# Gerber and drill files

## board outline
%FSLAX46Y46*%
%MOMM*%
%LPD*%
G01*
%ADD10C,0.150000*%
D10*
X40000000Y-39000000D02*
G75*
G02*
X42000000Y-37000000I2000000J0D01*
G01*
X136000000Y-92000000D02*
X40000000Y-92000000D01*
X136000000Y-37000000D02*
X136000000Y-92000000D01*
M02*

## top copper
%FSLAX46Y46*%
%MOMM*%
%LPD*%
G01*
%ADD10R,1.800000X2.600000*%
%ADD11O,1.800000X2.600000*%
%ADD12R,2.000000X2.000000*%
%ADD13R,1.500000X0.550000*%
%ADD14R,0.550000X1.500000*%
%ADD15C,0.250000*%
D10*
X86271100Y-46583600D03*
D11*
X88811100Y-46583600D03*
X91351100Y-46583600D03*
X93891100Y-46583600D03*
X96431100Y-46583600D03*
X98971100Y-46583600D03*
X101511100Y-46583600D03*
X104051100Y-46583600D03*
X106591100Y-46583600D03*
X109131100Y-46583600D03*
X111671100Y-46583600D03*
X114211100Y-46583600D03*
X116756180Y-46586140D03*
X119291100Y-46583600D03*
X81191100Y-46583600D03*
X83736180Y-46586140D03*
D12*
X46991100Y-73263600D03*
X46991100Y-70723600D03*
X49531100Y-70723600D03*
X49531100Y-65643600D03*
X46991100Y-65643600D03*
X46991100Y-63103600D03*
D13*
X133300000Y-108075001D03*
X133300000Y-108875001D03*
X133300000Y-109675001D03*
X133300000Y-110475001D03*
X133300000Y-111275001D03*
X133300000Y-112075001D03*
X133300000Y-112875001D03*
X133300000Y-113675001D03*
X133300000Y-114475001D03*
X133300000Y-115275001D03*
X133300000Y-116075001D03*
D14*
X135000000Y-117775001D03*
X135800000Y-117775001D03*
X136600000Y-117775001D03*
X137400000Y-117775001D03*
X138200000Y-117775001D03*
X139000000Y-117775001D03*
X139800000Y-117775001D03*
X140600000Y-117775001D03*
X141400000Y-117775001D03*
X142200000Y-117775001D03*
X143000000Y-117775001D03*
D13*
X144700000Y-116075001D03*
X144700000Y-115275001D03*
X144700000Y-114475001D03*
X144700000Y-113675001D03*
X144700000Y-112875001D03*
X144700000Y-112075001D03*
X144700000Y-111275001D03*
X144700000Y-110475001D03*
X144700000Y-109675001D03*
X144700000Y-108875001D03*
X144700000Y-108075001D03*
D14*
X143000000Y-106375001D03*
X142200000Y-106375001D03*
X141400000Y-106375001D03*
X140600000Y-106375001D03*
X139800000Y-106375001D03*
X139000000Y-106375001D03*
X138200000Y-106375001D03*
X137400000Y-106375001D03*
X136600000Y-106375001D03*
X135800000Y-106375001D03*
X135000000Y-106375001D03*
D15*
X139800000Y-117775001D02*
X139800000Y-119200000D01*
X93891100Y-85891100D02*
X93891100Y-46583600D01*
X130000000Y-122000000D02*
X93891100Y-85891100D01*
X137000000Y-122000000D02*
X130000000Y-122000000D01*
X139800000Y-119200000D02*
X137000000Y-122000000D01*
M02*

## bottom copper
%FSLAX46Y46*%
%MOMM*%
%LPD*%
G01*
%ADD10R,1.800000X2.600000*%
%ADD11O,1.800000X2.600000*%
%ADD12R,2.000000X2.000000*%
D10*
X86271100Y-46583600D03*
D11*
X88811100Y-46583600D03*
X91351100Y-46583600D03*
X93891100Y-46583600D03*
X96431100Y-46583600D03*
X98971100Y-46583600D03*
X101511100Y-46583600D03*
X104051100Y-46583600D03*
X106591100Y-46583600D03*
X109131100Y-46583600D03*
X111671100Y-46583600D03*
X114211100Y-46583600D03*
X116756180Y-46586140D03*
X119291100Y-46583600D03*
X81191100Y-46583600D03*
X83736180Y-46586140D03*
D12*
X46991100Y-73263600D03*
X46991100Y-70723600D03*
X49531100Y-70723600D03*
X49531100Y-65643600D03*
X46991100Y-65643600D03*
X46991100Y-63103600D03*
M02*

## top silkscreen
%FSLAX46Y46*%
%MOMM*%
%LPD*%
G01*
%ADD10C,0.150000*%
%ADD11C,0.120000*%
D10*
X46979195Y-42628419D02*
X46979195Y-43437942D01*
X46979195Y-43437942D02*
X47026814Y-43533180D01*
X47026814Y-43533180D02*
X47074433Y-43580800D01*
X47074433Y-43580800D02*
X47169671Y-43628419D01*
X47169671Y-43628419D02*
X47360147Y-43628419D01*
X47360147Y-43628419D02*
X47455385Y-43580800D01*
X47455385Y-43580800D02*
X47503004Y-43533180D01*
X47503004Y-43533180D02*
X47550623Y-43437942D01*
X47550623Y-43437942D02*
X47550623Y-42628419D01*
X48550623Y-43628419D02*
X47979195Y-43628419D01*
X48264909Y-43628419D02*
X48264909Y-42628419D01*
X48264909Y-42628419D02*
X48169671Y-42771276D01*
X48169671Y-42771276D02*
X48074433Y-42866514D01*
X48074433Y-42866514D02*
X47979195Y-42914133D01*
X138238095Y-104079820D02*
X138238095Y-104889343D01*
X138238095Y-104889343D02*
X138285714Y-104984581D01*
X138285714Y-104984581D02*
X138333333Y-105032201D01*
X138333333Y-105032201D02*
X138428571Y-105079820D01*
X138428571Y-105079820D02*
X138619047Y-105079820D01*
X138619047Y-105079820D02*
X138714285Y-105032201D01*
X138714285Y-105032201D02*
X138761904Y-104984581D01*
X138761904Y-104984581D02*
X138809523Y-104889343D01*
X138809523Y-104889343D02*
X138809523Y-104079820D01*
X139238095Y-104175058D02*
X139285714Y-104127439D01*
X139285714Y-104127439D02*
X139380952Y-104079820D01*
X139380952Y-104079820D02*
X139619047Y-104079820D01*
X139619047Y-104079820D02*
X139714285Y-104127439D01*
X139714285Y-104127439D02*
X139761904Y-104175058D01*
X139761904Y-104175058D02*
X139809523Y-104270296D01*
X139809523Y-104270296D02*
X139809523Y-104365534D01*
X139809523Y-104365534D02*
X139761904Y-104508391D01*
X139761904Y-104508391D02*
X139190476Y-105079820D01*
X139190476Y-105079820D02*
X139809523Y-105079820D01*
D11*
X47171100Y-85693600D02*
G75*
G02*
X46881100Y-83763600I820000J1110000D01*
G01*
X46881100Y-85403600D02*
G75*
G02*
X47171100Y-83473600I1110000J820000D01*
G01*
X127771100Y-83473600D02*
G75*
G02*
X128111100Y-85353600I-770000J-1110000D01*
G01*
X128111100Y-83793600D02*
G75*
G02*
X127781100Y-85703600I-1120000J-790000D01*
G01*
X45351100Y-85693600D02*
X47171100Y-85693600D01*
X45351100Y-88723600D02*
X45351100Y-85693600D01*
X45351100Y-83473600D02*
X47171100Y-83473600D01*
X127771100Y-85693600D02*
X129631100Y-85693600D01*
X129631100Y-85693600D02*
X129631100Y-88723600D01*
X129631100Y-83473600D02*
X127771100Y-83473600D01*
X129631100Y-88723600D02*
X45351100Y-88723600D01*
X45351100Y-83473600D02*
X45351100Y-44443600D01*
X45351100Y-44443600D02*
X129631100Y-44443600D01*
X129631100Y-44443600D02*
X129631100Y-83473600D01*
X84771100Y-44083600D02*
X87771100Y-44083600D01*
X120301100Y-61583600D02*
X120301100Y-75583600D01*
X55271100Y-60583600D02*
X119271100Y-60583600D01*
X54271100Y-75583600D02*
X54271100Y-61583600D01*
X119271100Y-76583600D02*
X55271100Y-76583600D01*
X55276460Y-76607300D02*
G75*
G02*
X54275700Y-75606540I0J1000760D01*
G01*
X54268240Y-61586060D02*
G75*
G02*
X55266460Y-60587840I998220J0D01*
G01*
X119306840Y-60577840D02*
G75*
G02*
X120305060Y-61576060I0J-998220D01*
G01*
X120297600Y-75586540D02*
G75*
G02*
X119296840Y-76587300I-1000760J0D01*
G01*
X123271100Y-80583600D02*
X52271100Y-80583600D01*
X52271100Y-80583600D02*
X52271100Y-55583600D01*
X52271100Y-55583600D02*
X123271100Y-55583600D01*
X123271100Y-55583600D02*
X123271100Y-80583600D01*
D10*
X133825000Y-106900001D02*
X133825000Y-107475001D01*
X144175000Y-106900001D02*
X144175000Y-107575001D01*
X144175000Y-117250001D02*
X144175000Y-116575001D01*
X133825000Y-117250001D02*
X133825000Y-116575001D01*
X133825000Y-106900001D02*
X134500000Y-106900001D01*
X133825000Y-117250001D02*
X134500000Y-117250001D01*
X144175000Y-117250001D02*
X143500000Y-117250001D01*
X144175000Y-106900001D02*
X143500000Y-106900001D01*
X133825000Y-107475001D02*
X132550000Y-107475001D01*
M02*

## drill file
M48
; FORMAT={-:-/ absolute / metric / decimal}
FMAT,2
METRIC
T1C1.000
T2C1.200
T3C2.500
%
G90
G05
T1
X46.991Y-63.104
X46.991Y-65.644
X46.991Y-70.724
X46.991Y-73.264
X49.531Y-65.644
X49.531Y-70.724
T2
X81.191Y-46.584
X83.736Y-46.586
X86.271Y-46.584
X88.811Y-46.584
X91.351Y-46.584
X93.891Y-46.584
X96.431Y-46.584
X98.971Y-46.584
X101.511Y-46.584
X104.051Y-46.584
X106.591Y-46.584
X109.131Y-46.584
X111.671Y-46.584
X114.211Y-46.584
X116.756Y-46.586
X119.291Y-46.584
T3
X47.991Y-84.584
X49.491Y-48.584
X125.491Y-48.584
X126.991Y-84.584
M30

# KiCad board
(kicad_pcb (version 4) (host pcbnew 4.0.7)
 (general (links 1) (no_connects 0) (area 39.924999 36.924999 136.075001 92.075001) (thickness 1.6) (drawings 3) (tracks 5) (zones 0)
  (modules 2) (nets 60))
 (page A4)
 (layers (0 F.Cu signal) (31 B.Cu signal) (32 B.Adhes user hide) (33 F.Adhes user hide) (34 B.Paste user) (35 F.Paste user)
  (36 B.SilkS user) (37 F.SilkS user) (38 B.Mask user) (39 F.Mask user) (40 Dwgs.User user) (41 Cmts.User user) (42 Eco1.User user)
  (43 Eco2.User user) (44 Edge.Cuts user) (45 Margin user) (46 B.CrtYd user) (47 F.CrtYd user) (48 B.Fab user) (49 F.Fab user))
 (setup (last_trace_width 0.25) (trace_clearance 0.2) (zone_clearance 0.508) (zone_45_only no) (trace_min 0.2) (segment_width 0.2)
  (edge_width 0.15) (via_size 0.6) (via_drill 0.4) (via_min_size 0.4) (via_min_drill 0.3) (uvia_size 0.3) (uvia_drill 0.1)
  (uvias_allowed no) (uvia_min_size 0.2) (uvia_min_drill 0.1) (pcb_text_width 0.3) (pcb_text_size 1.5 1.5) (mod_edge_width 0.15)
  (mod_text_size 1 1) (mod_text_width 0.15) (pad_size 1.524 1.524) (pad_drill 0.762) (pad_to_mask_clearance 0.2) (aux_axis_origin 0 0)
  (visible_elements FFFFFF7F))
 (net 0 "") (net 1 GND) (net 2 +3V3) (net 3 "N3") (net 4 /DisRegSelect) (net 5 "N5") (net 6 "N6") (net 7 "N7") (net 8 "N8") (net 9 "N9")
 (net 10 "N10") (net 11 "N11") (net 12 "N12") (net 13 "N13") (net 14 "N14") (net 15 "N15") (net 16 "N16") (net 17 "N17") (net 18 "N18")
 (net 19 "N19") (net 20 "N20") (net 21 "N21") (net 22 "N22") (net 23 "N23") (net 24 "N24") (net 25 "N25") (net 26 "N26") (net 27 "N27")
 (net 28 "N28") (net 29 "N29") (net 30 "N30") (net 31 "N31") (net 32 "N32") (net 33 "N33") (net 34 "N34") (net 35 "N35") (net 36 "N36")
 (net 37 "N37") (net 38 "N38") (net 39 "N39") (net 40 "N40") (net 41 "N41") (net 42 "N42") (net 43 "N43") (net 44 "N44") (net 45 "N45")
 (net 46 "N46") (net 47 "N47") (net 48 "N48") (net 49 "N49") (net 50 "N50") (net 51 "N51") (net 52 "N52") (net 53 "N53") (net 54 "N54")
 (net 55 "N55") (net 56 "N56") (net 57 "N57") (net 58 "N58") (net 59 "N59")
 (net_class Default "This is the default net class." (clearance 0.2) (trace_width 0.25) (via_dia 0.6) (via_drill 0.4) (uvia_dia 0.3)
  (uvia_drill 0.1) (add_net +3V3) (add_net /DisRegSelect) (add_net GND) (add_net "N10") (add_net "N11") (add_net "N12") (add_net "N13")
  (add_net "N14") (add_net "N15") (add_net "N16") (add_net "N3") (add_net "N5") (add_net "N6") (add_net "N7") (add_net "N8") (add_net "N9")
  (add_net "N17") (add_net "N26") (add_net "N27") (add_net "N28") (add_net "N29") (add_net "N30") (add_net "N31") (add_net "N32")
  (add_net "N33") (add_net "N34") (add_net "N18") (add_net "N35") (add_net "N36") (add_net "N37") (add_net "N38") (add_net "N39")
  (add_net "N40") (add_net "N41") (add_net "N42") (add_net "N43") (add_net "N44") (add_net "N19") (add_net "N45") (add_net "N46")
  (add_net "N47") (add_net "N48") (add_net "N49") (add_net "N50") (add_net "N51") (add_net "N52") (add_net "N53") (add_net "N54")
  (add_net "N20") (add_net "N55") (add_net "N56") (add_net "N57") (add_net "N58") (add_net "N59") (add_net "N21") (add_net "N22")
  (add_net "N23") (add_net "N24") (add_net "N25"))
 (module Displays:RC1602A (layer F.Cu) (at 86.2711 46.5836)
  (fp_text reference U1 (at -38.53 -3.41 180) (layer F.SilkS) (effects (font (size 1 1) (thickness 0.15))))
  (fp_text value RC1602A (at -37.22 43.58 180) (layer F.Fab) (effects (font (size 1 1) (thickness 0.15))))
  (fp_arc (start -38.28 38) (end -39.1 39.11) (angle 90) (layer F.SilkS) (width 0.12))
  (fp_arc (start -38.28 38) (end -39.39 38.82) (angle 90) (layer F.SilkS) (width 0.12))
  (fp_arc (start 40.73 38) (end 41.5 36.89) (angle 90) (layer F.SilkS) (width 0.12))
  (fp_arc (start 40.72 38) (end 41.84 37.21) (angle 90) (layer F.SilkS) (width 0.12))
  (fp_line (start -40.92 39.11) (end -39.1 39.11) (layer F.SilkS) (width 0.12))
  (fp_line (start -40.92 42.14) (end -40.92 39.11) (layer F.SilkS) (width 0.12))
  (fp_line (start -40.92 36.89) (end -39.1 36.89) (layer F.SilkS) (width 0.12))
  (fp_line (start 41.5 39.11) (end 43.36 39.11) (layer F.SilkS) (width 0.12))
  (fp_line (start 43.36 39.11) (end 43.36 42.14) (layer F.SilkS) (width 0.12))
  (fp_line (start 43.36 36.89) (end 41.5 36.89) (layer F.SilkS) (width 0.12))
  (fp_line (start 43.36 42.14) (end -40.92 42.14) (layer F.SilkS) (width 0.12))
  (fp_line (start -40.92 36.89) (end -40.92 -2.14) (layer F.SilkS) (width 0.12))
  (fp_line (start -40.92 -2.14) (end 43.36 -2.14) (layer F.SilkS) (width 0.12))
  (fp_line (start 43.36 -2.14) (end 43.36 36.89) (layer F.SilkS) (width 0.12))
  (fp_line (start -1.5 -2.5) (end 1.5 -2.5) (layer F.SilkS) (width 0.12))
  (fp_line (start 34.03 15) (end 34.03 29) (layer F.SilkS) (width 0.12))
  (fp_line (start -31 14) (end 33 14) (layer F.SilkS) (width 0.12))
  (fp_line (start -32 29) (end -32 15) (layer F.SilkS) (width 0.12))
  (fp_line (start 33 30) (end -31 30) (layer F.SilkS) (width 0.12))
  (fp_arc (start -30.99464 29.02294) (end -30.99464 30.0237) (angle 90) (layer F.SilkS) (width 0.12))
  (fp_arc (start -31.00464 15.00246) (end -32.00286 15.00246) (angle 90) (layer F.SilkS) (width 0.12))
  (fp_arc (start 33.03574 14.99246) (end 33.03574 13.99424) (angle 90) (layer F.SilkS) (width 0.12))
  (fp_arc (start 33.02574 29.00294) (end 34.0265 29.00294) (angle 90) (layer F.SilkS) (width 0.12))
  (fp_line (start 37 34) (end -34 34) (layer F.SilkS) (width 0.12))
  (fp_line (start -34 34) (end -34 9) (layer F.SilkS) (width 0.12))
  (fp_line (start -34 9) (end 37 9) (layer F.SilkS) (width 0.12))
  (fp_line (start 37 9) (end 37 34) (layer F.SilkS) (width 0.12))
  (pad 1 thru_hole rect (at 0 0 180) (size 1.8 2.6) (drill 1.2) (layers *.Cu *.Mask) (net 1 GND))
  (pad 2 thru_hole oval (at 2.54 0 180) (size 1.8 2.6) (drill 1.2) (layers *.Cu *.Mask) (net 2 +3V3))
  (pad 3 thru_hole oval (at 5.08 0 180) (size 1.8 2.6) (drill 1.2) (layers *.Cu *.Mask) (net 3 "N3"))
  (pad 4 thru_hole oval (at 7.62 0 180) (size 1.8 2.6) (drill 1.2) (layers *.Cu *.Mask) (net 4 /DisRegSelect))
  (pad 5 thru_hole oval (at 10.16 0 180) (size 1.8 2.6) (drill 1.2) (layers *.Cu *.Mask) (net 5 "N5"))
  (pad 6 thru_hole oval (at 12.7 0 180) (size 1.8 2.6) (drill 1.2) (layers *.Cu *.Mask) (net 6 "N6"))
  (pad 7 thru_hole oval (at 15.24 0 180) (size 1.8 2.6) (drill 1.2) (layers *.Cu *.Mask) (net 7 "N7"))
  (pad 8 thru_hole oval (at 17.78 0 180) (size 1.8 2.6) (drill 1.2) (layers *.Cu *.Mask) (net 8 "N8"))
  (pad 9 thru_hole oval (at 20.32 0 180) (size 1.8 2.6) (drill 1.2) (layers *.Cu *.Mask) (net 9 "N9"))
  (pad 10 thru_hole oval (at 22.86 0 180) (size 1.8 2.6) (drill 1.2) (layers *.Cu *.Mask) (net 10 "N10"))
  (pad 11 thru_hole oval (at 25.4 0 180) (size 1.8 2.6) (drill 1.2) (layers *.Cu *.Mask) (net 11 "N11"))
  (pad 12 thru_hole oval (at 27.94 0 180) (size 1.8 2.6) (drill 1.2) (layers *.Cu *.Mask) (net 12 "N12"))
  (pad 13 thru_hole oval (at 30.48508 0.00254 180) (size 1.8 2.6) (drill 1.2) (layers *.Cu *.Mask) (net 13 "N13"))
  (pad 14 thru_hole oval (at 33.02 0 180) (size 1.8 2.6) (drill 1.2) (layers *.Cu *.Mask) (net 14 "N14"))
  (pad 15 thru_hole oval (at -5.08 0 180) (size 1.8 2.6) (drill 1.2) (layers *.Cu *.Mask) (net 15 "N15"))
  (pad 16 thru_hole oval (at -2.53492 0.00254 180) (size 1.8 2.6) (drill 1.2) (layers *.Cu *.Mask) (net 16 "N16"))
  (pad "" np_thru_hole circle (at 39.22 2 180) (size 2.5 2.5) (drill 2.5) (layers *.Cu *.Mask))
  (pad "" np_thru_hole circle (at 40.72 38 180) (size 2.5 2.5) (drill 2.5) (layers *.Cu *.Mask))
  (pad "" np_thru_hole circle (at -38.28 38 180) (size 2.5 2.5) (drill 2.5) (layers *.Cu *.Mask))
  (pad "" np_thru_hole circle (at -36.78 2 180) (size 2.5 2.5) (drill 2.5) (layers *.Cu *.Mask))
  (pad A1 thru_hole rect (at -39.28 26.68 180) (size 2 2) (drill 1) (layers *.Cu *.Mask))
  (pad A1 thru_hole rect (at -39.28 24.14 180) (size 2 2) (drill 1) (layers *.Cu *.Mask))
  (pad A1 thru_hole rect (at -36.74 24.14 180) (size 2 2) (drill 1) (layers *.Cu *.Mask))
  (pad K1 thru_hole rect (at -36.74 19.06 180) (size 2 2) (drill 1) (layers *.Cu *.Mask))
  (pad K1 thru_hole rect (at -39.28 19.06 180) (size 2 2) (drill 1) (layers *.Cu *.Mask))
  (pad K1 thru_hole rect (at -39.28 16.52 180) (size 2 2) (drill 1) (layers *.Cu *.Mask)))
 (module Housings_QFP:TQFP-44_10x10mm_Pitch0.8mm (layer F.Cu) (at 139 112.075001)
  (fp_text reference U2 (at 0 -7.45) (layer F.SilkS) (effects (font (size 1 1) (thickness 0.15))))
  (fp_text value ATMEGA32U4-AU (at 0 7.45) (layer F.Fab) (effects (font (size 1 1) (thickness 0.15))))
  (fp_line (start -5.175 -5.175) (end -5.175 -4.6) (layer F.SilkS) (width 0.15))
  (fp_line (start 5.175 -5.175) (end 5.175 -4.5) (layer F.SilkS) (width 0.15))
  (fp_line (start 5.175 5.175) (end 5.175 4.5) (layer F.SilkS) (width 0.15))
  (fp_line (start -5.175 5.175) (end -5.175 4.5) (layer F.SilkS) (width 0.15))
  (fp_line (start -5.175 -5.175) (end -4.5 -5.175) (layer F.SilkS) (width 0.15))
  (fp_line (start -5.175 5.175) (end -4.5 5.175) (layer F.SilkS) (width 0.15))
  (fp_line (start 5.175 5.175) (end 4.5 5.175) (layer F.SilkS) (width 0.15))
  (fp_line (start 5.175 -5.175) (end 4.5 -5.175) (layer F.SilkS) (width 0.15))
  (fp_line (start -5.175 -4.6) (end -6.45 -4.6) (layer F.SilkS) (width 0.15))
  (pad 1 smd rect (at -5.7 -4) (size 1.5 0.55) (layers F.Cu F.Paste F.Mask) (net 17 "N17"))
  (pad 2 smd rect (at -5.7 -3.2) (size 1.5 0.55) (layers F.Cu F.Paste F.Mask) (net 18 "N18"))
  (pad 3 smd rect (at -5.7 -2.4) (size 1.5 0.55) (layers F.Cu F.Paste F.Mask) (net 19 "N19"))
  (pad 4 smd rect (at -5.7 -1.6) (size 1.5 0.55) (layers F.Cu F.Paste F.Mask) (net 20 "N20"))
  (pad 5 smd rect (at -5.7 -0.8) (size 1.5 0.55) (layers F.Cu F.Paste F.Mask) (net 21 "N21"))
  (pad 6 smd rect (at -5.7 0) (size 1.5 0.55) (layers F.Cu F.Paste F.Mask) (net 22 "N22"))
  (pad 7 smd rect (at -5.7 0.8) (size 1.5 0.55) (layers F.Cu F.Paste F.Mask) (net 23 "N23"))
  (pad 8 smd rect (at -5.7 1.6) (size 1.5 0.55) (layers F.Cu F.Paste F.Mask) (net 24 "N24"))
  (pad 9 smd rect (at -5.7 2.4) (size 1.5 0.55) (layers F.Cu F.Paste F.Mask) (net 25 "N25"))
  (pad 10 smd rect (at -5.7 3.2) (size 1.5 0.55) (layers F.Cu F.Paste F.Mask) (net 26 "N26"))
  (pad 11 smd rect (at -5.7 4) (size 1.5 0.55) (layers F.Cu F.Paste F.Mask) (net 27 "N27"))
  (pad 12 smd rect (at -4 5.7 90) (size 1.5 0.55) (layers F.Cu F.Paste F.Mask) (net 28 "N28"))
  (pad 13 smd rect (at -3.2 5.7 90) (size 1.5 0.55) (layers F.Cu F.Paste F.Mask) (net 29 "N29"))
  (pad 14 smd rect (at -2.4 5.7 90) (size 1.5 0.55) (layers F.Cu F.Paste F.Mask) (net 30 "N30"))
  (pad 15 smd rect (at -1.6 5.7 90) (size 1.5 0.55) (layers F.Cu F.Paste F.Mask) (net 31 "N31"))
  (pad 16 smd rect (at -0.8 5.7 90) (size 1.5 0.55) (layers F.Cu F.Paste F.Mask) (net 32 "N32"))
  (pad 17 smd rect (at 0 5.7 90) (size 1.5 0.55) (layers F.Cu F.Paste F.Mask) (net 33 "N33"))
  (pad 18 smd rect (at 0.8 5.7 90) (size 1.5 0.55) (layers F.Cu F.Paste F.Mask) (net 4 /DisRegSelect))
  (pad 19 smd rect (at 1.6 5.7 90) (size 1.5 0.55) (layers F.Cu F.Paste F.Mask) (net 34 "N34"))
  (pad 20 smd rect (at 2.4 5.7 90) (size 1.5 0.55) (layers F.Cu F.Paste F.Mask) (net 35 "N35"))
  (pad 21 smd rect (at 3.2 5.7 90) (size 1.5 0.55) (layers F.Cu F.Paste F.Mask) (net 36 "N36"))
  (pad 22 smd rect (at 4 5.7 90) (size 1.5 0.55) (layers F.Cu F.Paste F.Mask) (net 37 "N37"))
  (pad 23 smd rect (at 5.7 4) (size 1.5 0.55) (layers F.Cu F.Paste F.Mask) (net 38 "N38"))
  (pad 24 smd rect (at 5.7 3.2) (size 1.5 0.55) (layers F.Cu F.Paste F.Mask) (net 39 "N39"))
  (pad 25 smd rect (at 5.7 2.4) (size 1.5 0.55) (layers F.Cu F.Paste F.Mask) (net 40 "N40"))
  (pad 26 smd rect (at 5.7 1.6) (size 1.5 0.55) (layers F.Cu F.Paste F.Mask) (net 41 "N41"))
  (pad 27 smd rect (at 5.7 0.8) (size 1.5 0.55) (layers F.Cu F.Paste F.Mask) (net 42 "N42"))
  (pad 28 smd rect (at 5.7 0) (size 1.5 0.55) (layers F.Cu F.Paste F.Mask) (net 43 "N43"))
  (pad 29 smd rect (at 5.7 -0.8) (size 1.5 0.55) (layers F.Cu F.Paste F.Mask) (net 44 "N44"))
  (pad 30 smd rect (at 5.7 -1.6) (size 1.5 0.55) (layers F.Cu F.Paste F.Mask) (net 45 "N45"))
  (pad 31 smd rect (at 5.7 -2.4) (size 1.5 0.55) (layers F.Cu F.Paste F.Mask) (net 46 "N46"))
  (pad 32 smd rect (at 5.7 -3.2) (size 1.5 0.55) (layers F.Cu F.Paste F.Mask) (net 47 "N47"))
  (pad 33 smd rect (at 5.7 -4) (size 1.5 0.55) (layers F.Cu F.Paste F.Mask) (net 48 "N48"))
  (pad 34 smd rect (at 4 -5.7 90) (size 1.5 0.55) (layers F.Cu F.Paste F.Mask) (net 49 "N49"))
  (pad 35 smd rect (at 3.2 -5.7 90) (size 1.5 0.55) (layers F.Cu F.Paste F.Mask) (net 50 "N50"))
  (pad 36 smd rect (at 2.4 -5.7 90) (size 1.5 0.55) (layers F.Cu F.Paste F.Mask) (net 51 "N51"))
  (pad 37 smd rect (at 1.6 -5.7 90) (size 1.5 0.55) (layers F.Cu F.Paste F.Mask) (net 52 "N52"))
  (pad 38 smd rect (at 0.8 -5.7 90) (size 1.5 0.55) (layers F.Cu F.Paste F.Mask) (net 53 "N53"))
  (pad 39 smd rect (at 0 -5.7 90) (size 1.5 0.55) (layers F.Cu F.Paste F.Mask) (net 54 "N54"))
  (pad 40 smd rect (at -0.8 -5.7 90) (size 1.5 0.55) (layers F.Cu F.Paste F.Mask) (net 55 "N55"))
  (pad 41 smd rect (at -1.6 -5.7 90) (size 1.5 0.55) (layers F.Cu F.Paste F.Mask) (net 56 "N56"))
  (pad 42 smd rect (at -2.4 -5.7 90) (size 1.5 0.55) (layers F.Cu F.Paste F.Mask) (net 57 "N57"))
  (pad 43 smd rect (at -3.2 -5.7 90) (size 1.5 0.55) (layers F.Cu F.Paste F.Mask) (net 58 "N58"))
  (pad 44 smd rect (at -4 -5.7 90) (size 1.5 0.55) (layers F.Cu F.Paste F.Mask) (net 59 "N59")))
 (gr_arc (start 42 39) (end 40 39) (angle 90) (layer Edge.Cuts) (width 0.15))
 (gr_line (start 136 92) (end 40 92) (angle 90) (layer Edge.Cuts) (width 0.15))
 (gr_line (start 136 37) (end 136 92) (angle 90) (layer Edge.Cuts) (width 0.15))
 (segment (start 139.8 117.775001) (end 139.8 119.2) (width 0.25) (layer F.Cu) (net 4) (status 400000))
 (segment (start 93.8911 85.8911) (end 93.8911 46.5836) (width 0.25) (layer F.Cu) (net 4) (status 800000))
 (segment (start 130 122) (end 93.8911 85.8911) (width 0.25) (layer F.Cu) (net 4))
 (segment (start 137 122) (end 130 122) (width 0.25) (layer F.Cu) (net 4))
 (segment (start 139.8 119.2) (end 137 122) (width 0.25) (layer F.Cu) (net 4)))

